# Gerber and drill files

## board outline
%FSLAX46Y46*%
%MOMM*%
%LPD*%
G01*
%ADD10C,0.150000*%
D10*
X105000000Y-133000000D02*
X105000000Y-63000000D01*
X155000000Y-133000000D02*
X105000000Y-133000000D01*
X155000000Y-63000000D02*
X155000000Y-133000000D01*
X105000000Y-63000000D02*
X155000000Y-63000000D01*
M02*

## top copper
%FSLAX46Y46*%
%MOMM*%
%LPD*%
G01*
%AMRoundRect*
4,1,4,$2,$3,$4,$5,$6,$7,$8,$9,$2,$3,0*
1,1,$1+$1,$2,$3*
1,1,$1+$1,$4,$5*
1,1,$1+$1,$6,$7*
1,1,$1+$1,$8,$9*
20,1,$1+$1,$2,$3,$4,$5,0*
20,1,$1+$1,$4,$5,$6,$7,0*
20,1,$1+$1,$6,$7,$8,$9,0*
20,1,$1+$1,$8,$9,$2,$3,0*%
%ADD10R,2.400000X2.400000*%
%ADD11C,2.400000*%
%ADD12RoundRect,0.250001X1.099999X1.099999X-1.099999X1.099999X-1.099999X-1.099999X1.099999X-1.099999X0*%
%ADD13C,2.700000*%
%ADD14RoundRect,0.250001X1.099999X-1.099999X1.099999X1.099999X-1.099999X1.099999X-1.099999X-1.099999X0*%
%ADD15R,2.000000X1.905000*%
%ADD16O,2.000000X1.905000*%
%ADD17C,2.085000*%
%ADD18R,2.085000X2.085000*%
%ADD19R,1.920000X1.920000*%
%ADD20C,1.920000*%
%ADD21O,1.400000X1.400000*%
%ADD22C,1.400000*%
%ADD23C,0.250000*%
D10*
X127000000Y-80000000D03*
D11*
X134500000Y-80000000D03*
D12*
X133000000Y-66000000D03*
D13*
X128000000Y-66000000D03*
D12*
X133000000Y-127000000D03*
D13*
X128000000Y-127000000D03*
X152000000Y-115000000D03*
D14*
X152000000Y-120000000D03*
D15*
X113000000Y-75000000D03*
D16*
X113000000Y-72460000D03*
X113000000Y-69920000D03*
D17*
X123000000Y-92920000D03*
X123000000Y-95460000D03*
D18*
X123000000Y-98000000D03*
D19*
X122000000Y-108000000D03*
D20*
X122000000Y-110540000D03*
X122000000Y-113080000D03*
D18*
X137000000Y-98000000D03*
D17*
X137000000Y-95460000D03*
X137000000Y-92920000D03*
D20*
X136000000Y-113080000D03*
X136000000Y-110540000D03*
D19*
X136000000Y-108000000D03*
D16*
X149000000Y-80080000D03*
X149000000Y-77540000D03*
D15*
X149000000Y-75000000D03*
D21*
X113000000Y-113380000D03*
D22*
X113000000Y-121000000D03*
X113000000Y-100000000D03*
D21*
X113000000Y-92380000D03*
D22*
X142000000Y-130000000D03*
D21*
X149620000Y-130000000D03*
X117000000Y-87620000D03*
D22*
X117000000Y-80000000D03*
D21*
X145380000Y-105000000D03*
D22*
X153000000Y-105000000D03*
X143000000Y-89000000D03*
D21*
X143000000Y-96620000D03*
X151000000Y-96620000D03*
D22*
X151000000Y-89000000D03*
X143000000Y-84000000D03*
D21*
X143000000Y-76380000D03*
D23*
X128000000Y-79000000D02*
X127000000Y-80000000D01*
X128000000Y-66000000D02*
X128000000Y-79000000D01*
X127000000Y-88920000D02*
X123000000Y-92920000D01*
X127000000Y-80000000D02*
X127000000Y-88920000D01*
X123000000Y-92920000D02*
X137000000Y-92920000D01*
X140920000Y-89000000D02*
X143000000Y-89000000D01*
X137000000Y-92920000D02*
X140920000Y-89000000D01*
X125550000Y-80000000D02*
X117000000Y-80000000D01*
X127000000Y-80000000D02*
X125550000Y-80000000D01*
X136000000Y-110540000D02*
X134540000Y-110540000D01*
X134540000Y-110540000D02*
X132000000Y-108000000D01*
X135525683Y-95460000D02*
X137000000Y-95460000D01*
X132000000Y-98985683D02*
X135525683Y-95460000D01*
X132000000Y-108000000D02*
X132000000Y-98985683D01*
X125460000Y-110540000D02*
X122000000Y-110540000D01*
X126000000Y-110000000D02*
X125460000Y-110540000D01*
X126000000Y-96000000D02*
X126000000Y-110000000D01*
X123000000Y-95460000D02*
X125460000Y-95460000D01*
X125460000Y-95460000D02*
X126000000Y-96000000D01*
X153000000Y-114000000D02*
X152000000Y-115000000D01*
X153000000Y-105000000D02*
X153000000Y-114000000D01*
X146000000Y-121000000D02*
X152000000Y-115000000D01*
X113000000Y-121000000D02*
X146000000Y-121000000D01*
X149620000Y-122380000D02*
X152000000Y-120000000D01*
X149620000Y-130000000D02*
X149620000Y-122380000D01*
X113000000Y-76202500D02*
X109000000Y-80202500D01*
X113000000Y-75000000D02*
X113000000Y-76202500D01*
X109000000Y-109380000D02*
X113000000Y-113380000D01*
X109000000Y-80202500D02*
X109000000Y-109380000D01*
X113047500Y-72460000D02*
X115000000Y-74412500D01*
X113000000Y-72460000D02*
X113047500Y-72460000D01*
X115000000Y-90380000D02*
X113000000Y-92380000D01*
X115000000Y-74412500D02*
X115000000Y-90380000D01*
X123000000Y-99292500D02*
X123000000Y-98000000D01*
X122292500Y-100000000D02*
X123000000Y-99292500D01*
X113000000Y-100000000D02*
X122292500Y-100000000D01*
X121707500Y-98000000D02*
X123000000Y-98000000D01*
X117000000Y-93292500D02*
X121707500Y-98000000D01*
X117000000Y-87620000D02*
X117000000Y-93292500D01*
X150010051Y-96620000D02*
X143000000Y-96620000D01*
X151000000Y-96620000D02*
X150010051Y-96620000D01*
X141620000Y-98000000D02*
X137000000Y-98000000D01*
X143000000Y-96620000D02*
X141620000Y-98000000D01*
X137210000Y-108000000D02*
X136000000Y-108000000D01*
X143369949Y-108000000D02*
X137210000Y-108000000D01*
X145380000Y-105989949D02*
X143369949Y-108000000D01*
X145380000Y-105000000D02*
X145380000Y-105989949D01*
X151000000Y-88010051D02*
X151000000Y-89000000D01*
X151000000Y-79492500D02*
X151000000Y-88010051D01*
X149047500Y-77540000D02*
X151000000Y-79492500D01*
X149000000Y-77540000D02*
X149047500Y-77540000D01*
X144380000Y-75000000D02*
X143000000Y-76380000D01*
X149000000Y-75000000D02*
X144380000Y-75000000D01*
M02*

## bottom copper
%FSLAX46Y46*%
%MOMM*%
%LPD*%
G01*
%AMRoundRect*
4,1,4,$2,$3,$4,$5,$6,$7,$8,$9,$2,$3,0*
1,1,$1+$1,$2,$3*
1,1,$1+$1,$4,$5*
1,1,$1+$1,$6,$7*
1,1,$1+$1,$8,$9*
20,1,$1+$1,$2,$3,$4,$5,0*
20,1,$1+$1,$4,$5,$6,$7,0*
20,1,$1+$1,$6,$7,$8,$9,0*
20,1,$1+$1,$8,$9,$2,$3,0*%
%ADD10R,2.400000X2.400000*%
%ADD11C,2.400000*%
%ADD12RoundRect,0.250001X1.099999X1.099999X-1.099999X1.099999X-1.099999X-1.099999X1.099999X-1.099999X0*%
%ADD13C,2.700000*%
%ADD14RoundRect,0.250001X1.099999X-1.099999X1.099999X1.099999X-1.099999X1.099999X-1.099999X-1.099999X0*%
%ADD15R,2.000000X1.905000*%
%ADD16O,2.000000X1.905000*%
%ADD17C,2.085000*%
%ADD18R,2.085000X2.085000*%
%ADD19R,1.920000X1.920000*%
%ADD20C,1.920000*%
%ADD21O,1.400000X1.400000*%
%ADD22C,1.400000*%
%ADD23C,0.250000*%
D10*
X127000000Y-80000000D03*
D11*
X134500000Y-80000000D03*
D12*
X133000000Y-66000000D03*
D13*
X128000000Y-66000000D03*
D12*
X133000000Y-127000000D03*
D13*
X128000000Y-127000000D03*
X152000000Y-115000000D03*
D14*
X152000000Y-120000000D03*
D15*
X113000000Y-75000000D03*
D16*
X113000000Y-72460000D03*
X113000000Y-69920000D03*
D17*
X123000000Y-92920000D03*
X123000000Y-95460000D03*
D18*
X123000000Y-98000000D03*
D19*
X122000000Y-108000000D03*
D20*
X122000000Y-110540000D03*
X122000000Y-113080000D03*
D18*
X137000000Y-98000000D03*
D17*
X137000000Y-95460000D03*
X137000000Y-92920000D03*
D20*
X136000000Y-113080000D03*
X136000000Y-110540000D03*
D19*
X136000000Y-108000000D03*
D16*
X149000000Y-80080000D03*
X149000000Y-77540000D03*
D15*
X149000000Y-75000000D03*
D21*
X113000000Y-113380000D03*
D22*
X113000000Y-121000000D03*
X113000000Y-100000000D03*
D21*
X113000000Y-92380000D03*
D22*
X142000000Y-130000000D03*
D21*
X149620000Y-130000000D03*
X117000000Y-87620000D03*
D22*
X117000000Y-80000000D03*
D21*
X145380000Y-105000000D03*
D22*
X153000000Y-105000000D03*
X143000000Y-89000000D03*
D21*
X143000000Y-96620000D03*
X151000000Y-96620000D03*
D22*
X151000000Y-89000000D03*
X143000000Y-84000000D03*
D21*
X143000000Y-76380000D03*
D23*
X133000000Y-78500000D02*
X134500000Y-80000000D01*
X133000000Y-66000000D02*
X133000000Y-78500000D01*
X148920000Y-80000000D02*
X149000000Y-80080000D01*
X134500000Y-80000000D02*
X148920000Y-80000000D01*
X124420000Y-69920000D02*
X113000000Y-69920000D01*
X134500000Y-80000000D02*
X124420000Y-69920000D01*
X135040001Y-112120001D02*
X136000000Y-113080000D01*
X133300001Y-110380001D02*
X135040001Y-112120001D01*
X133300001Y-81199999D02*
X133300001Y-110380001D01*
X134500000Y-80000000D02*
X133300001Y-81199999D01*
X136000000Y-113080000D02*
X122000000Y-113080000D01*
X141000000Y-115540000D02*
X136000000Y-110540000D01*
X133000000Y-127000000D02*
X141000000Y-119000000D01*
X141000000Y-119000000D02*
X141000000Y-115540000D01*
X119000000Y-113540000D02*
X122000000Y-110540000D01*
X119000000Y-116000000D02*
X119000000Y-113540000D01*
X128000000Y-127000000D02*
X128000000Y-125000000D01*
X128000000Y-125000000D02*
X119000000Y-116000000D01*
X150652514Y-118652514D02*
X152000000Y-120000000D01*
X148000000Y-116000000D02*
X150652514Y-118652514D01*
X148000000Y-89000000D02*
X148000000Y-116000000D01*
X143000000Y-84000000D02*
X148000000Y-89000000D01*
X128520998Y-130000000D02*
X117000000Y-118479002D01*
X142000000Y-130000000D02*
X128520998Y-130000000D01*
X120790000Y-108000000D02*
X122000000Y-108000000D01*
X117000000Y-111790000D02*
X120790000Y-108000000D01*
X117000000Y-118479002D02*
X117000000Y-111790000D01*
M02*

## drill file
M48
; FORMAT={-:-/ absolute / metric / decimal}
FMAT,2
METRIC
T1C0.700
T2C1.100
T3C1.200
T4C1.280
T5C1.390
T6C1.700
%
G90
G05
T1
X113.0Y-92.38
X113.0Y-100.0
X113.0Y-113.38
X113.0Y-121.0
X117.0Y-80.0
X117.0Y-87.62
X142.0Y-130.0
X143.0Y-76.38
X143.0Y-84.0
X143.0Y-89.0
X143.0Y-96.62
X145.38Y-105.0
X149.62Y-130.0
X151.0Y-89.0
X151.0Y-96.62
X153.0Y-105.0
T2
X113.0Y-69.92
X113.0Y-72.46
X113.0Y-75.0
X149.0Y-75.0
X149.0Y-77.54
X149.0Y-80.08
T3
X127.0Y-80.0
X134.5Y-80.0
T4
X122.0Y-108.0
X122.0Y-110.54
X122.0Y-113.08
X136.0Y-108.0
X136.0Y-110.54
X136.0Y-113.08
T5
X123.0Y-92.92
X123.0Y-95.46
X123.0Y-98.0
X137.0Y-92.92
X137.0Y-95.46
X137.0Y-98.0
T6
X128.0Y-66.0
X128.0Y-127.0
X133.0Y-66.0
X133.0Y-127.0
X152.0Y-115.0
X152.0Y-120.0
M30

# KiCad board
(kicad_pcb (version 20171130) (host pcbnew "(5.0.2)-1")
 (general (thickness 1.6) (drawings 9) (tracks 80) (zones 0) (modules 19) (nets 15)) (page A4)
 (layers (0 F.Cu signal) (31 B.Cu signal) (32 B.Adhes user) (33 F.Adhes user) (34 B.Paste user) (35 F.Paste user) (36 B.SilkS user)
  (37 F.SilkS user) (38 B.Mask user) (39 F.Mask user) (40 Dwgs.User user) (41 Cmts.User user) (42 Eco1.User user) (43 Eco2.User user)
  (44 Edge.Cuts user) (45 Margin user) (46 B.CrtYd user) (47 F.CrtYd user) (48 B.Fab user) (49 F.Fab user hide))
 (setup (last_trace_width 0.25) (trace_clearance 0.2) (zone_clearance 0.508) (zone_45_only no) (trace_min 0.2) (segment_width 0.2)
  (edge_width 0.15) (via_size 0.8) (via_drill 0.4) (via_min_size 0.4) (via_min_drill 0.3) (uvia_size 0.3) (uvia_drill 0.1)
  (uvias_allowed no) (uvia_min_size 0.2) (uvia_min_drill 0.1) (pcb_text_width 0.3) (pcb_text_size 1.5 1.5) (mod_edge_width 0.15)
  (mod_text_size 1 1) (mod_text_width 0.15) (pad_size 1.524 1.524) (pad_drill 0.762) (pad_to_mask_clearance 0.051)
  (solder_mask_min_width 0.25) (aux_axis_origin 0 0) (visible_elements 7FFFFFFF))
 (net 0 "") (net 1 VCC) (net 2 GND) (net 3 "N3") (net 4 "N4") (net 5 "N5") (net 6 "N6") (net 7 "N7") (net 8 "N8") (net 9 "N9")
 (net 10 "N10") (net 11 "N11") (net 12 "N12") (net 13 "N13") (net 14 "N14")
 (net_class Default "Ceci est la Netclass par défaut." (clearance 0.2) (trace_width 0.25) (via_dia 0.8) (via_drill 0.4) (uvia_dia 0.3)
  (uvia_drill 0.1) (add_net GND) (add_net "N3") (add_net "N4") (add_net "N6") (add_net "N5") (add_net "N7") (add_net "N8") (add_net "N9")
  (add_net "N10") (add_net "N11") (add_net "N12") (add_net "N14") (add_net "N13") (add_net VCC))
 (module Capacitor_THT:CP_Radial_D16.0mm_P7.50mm (layer F.Cu) (at 127 80)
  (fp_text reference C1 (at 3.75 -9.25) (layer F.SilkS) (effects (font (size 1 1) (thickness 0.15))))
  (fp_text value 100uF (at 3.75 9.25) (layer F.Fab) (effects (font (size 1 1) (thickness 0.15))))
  (pad 1 thru_hole rect (at 0 0) (size 2.4 2.4) (drill 1.2) (layers *.Cu *.Mask) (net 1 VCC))
  (pad 2 thru_hole circle (at 7.5 0) (size 2.4 2.4) (drill 1.2) (layers *.Cu *.Mask) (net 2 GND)))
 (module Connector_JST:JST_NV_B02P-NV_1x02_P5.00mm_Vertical (layer F.Cu) (at 133 66 180)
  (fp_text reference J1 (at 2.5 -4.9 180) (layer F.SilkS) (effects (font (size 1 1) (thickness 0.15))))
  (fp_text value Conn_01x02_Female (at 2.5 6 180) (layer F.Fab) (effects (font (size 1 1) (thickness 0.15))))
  (pad 1 thru_hole roundrect (at 0 0 180) (size 2.7 2.7) (drill 1.7) (layers *.Cu *.Mask) (roundrect_rratio 0.09259299999999999) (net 2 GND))
  (pad 2 thru_hole circle (at 5 0 180) (size 2.7 2.7) (drill 1.7) (layers *.Cu *.Mask) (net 1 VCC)))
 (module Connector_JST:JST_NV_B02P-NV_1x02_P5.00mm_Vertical (layer F.Cu) (at 133 127 180)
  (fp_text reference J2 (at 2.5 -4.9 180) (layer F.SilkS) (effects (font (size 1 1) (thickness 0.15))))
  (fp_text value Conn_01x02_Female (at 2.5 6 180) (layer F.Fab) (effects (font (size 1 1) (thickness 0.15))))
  (pad 1 thru_hole roundrect (at 0 0 180) (size 2.7 2.7) (drill 1.7) (layers *.Cu *.Mask) (roundrect_rratio 0.09259299999999999)
   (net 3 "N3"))
  (pad 2 thru_hole circle (at 5 0 180) (size 2.7 2.7) (drill 1.7) (layers *.Cu *.Mask) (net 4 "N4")))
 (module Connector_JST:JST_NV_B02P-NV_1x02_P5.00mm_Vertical (layer F.Cu) (at 152 120 90)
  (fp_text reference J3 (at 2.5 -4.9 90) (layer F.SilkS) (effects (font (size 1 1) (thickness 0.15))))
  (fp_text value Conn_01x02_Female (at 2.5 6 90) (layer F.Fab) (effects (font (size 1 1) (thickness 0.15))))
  (pad 2 thru_hole circle (at 5 0 90) (size 2.7 2.7) (drill 1.7) (layers *.Cu *.Mask) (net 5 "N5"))
  (pad 1 thru_hole roundrect (at 0 0 90) (size 2.7 2.7) (drill 1.7) (layers *.Cu *.Mask) (roundrect_rratio 0.09259299999999999) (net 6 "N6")))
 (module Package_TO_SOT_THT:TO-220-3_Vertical (layer F.Cu) (at 113 75 90)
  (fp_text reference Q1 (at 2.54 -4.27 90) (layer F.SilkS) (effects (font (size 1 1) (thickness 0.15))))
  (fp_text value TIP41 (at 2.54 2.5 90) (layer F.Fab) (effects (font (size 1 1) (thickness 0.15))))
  (pad 1 thru_hole rect (at 0 0 90) (size 1.905 2) (drill 1.1) (layers *.Cu *.Mask) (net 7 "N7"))
  (pad 2 thru_hole oval (at 2.54 0 90) (size 1.905 2) (drill 1.1) (layers *.Cu *.Mask) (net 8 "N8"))
  (pad 3 thru_hole oval (at 5.08 0 90) (size 1.905 2) (drill 1.1) (layers *.Cu *.Mask) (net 2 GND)))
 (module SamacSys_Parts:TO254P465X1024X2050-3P (layer F.Cu) (at 123 98 90)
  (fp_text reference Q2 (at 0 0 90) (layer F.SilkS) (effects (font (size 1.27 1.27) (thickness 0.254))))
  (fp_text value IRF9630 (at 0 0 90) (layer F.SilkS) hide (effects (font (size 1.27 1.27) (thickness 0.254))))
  (pad 3 thru_hole circle (at 5.08 0 90) (size 2.085 2.085) (drill 1.39) (layers *.Cu *.Mask) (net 1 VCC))
  (pad 2 thru_hole circle (at 2.54 0 90) (size 2.085 2.085) (drill 1.39) (layers *.Cu *.Mask) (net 4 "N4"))
  (pad 1 thru_hole rect (at 0 0 90) (size 2.085 2.085) (drill 1.39) (layers *.Cu *.Mask) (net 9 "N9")))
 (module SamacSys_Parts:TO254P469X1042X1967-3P (layer F.Cu) (at 122 108 270)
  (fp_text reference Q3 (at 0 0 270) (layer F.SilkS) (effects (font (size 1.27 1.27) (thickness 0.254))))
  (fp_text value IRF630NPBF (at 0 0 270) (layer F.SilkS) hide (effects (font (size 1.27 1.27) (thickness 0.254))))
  (pad 1 thru_hole rect (at 0 0 270) (size 1.92 1.92) (drill 1.28) (layers *.Cu *.Mask) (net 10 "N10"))
  (pad 2 thru_hole circle (at 2.54 0 270) (size 1.92 1.92) (drill 1.28) (layers *.Cu *.Mask) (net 4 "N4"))
  (pad 3 thru_hole circle (at 5.08 0 270) (size 1.92 1.92) (drill 1.28) (layers *.Cu *.Mask) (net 2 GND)))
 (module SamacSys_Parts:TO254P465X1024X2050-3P (layer F.Cu) (at 137 98 90)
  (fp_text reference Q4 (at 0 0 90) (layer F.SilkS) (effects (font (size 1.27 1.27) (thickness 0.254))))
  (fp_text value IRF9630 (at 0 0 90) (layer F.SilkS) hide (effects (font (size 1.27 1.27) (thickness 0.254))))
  (pad 1 thru_hole rect (at 0 0 90) (size 2.085 2.085) (drill 1.39) (layers *.Cu *.Mask) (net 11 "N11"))
  (pad 2 thru_hole circle (at 2.54 0 90) (size 2.085 2.085) (drill 1.39) (layers *.Cu *.Mask) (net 3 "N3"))
  (pad 3 thru_hole circle (at 5.08 0 90) (size 2.085 2.085) (drill 1.39) (layers *.Cu *.Mask) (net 1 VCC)))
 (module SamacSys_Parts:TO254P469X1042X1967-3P (layer F.Cu) (at 136 108 270)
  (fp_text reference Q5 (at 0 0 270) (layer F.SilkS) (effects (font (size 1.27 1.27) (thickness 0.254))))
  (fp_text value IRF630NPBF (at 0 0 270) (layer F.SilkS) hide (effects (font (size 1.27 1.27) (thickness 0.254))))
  (pad 3 thru_hole circle (at 5.08 0 270) (size 1.92 1.92) (drill 1.28) (layers *.Cu *.Mask) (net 2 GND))
  (pad 2 thru_hole circle (at 2.54 0 270) (size 1.92 1.92) (drill 1.28) (layers *.Cu *.Mask) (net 3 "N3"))
  (pad 1 thru_hole rect (at 0 0 270) (size 1.92 1.92) (drill 1.28) (layers *.Cu *.Mask) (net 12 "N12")))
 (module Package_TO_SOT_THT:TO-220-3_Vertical (layer F.Cu) (at 149 75 270)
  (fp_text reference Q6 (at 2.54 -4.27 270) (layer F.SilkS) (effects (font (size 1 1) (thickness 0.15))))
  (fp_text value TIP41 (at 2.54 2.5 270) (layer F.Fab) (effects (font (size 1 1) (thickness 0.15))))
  (pad 3 thru_hole oval (at 5.08 0 270) (size 1.905 2) (drill 1.1) (layers *.Cu *.Mask) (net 2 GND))
  (pad 2 thru_hole oval (at 2.54 0 270) (size 1.905 2) (drill 1.1) (layers *.Cu *.Mask) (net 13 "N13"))
  (pad 1 thru_hole rect (at 0 0 270) (size 1.905 2) (drill 1.1) (layers *.Cu *.Mask) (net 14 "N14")))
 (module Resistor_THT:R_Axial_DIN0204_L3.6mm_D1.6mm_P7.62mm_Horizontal (layer F.Cu) (at 113 121 90)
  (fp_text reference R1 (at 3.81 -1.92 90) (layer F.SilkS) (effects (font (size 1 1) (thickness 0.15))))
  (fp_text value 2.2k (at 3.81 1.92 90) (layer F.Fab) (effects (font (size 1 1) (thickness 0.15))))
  (pad 2 thru_hole oval (at 7.62 0 90) (size 1.4 1.4) (drill 0.7) (layers *.Cu *.Mask) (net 7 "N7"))
  (pad 1 thru_hole circle (at 0 0 90) (size 1.4 1.4) (drill 0.7) (layers *.Cu *.Mask) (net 5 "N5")))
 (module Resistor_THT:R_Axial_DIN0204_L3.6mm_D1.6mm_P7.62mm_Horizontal (layer F.Cu) (at 113 100 90)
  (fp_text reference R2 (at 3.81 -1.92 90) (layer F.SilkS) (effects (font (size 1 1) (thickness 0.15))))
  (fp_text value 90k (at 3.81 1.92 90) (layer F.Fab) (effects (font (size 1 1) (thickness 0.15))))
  (pad 1 thru_hole circle (at 0 0 90) (size 1.4 1.4) (drill 0.7) (layers *.Cu *.Mask) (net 9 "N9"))
  (pad 2 thru_hole oval (at 7.62 0 90) (size 1.4 1.4) (drill 0.7) (layers *.Cu *.Mask) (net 8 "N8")))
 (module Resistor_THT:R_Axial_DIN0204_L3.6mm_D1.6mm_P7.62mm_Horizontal (layer F.Cu) (at 142 130)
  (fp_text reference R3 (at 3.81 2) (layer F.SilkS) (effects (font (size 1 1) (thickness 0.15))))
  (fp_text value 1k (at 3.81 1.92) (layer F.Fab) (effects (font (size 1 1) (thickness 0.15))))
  (pad 1 thru_hole circle (at 0 0) (size 1.4 1.4) (drill 0.7) (layers *.Cu *.Mask) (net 10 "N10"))
  (pad 2 thru_hole oval (at 7.62 0) (size 1.4 1.4) (drill 0.7) (layers *.Cu *.Mask) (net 6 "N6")))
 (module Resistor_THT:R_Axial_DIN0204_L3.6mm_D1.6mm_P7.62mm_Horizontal (layer F.Cu) (at 117 80 270)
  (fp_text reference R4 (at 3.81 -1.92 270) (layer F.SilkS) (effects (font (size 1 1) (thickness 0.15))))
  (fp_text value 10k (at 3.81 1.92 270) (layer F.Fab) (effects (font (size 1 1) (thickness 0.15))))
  (pad 2 thru_hole oval (at 7.62 0 270) (size 1.4 1.4) (drill 0.7) (layers *.Cu *.Mask) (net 9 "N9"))
  (pad 1 thru_hole circle (at 0 0 270) (size 1.4 1.4) (drill 0.7) (layers *.Cu *.Mask) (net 1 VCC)))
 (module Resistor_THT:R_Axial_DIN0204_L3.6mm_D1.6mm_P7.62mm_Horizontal (layer F.Cu) (at 153 105 180)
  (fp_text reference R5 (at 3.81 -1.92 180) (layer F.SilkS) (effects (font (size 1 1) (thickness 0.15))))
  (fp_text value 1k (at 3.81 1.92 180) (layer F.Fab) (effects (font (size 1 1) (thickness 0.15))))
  (pad 2 thru_hole oval (at 7.62 0 180) (size 1.4 1.4) (drill 0.7) (layers *.Cu *.Mask) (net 12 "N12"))
  (pad 1 thru_hole circle (at 0 0 180) (size 1.4 1.4) (drill 0.7) (layers *.Cu *.Mask) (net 5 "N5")))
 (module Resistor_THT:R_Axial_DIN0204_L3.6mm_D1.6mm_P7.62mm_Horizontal (layer F.Cu) (at 143 89 270)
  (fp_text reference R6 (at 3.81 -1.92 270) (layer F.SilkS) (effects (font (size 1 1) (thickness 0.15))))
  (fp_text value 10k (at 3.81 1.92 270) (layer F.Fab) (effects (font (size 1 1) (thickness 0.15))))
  (pad 1 thru_hole circle (at 0 0 270) (size 1.4 1.4) (drill 0.7) (layers *.Cu *.Mask) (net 1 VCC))
  (pad 2 thru_hole oval (at 7.62 0 270) (size 1.4 1.4) (drill 0.7) (layers *.Cu *.Mask) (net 11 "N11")))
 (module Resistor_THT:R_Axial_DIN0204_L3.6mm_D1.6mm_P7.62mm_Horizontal (layer F.Cu) (at 151 89 270)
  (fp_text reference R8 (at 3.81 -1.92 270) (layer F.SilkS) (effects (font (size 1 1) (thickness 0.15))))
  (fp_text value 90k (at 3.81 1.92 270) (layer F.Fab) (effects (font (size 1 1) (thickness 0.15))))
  (pad 2 thru_hole oval (at 7.62 0 270) (size 1.4 1.4) (drill 0.7) (layers *.Cu *.Mask) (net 11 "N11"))
  (pad 1 thru_hole circle (at 0 0 270) (size 1.4 1.4) (drill 0.7) (layers *.Cu *.Mask) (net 13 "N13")))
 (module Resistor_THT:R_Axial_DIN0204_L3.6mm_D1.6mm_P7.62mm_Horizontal (layer F.Cu) (at 143 84 90)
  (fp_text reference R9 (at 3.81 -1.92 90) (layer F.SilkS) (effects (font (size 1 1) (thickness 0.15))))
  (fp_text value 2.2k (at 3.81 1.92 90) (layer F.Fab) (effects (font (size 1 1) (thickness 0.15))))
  (pad 1 thru_hole circle (at 0 0 90) (size 1.4 1.4) (drill 0.7) (layers *.Cu *.Mask) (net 6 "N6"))
  (pad 2 thru_hole oval (at 7.62 0 90) (size 1.4 1.4) (drill 0.7) (layers *.Cu *.Mask) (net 14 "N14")))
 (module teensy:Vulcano (layer F.Cu) (at 125 127)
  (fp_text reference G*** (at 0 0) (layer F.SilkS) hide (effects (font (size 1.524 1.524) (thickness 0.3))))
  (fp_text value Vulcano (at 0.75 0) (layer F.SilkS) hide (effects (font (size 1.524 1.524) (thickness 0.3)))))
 (gr_line (start 105 133) (end 105 63) (layer Edge.Cuts) (width 0.15))
 (gr_line (start 155 133) (end 105 133) (layer Edge.Cuts) (width 0.15))
 (gr_line (start 155 63) (end 155 133) (layer Edge.Cuts) (width 0.15))
 (gr_line (start 105 63) (end 155 63) (layer Edge.Cuts) (width 0.15))
 (segment (start 128 79) (end 127 80) (width 0.25) (layer F.Cu) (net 1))
 (segment (start 128 66) (end 128 79) (width 0.25) (layer F.Cu) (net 1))
 (segment (start 127 88.92) (end 123 92.92) (width 0.25) (layer F.Cu) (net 1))
 (segment (start 127 80) (end 127 88.92) (width 0.25) (layer F.Cu) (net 1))
 (segment (start 123 92.92) (end 137 92.92) (width 0.25) (layer F.Cu) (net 1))
 (segment (start 140.92 89) (end 143 89) (width 0.25) (layer F.Cu) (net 1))
 (segment (start 137 92.92) (end 140.92 89) (width 0.25) (layer F.Cu) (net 1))
 (segment (start 125.55 80) (end 117 80) (width 0.25) (layer F.Cu) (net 1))
 (segment (start 127 80) (end 125.55 80) (width 0.25) (layer F.Cu) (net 1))
 (segment (start 133 78.5) (end 134.5 80) (width 0.25) (layer B.Cu) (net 2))
 (segment (start 133 66) (end 133 78.5) (width 0.25) (layer B.Cu) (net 2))
 (segment (start 148.92 80) (end 149 80.08) (width 0.25) (layer B.Cu) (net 2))
 (segment (start 134.5 80) (end 148.92 80) (width 0.25) (layer B.Cu) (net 2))
 (segment (start 124.42 69.92) (end 113 69.92) (width 0.25) (layer B.Cu) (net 2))
 (segment (start 134.5 80) (end 124.42 69.92) (width 0.25) (layer B.Cu) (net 2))
 (segment (start 135.040001 112.120001) (end 136 113.08) (width 0.25) (layer B.Cu) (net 2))
 (segment (start 133.300001 110.380001) (end 135.040001 112.120001) (width 0.25) (layer B.Cu) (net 2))
 (segment (start 133.300001 81.199999) (end 133.300001 110.380001) (width 0.25) (layer B.Cu) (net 2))
 (segment (start 134.5 80) (end 133.300001 81.199999) (width 0.25) (layer B.Cu) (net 2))
 (segment (start 136 113.08) (end 122 113.08) (width 0.25) (layer B.Cu) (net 2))
 (segment (start 136 110.54) (end 134.54 110.54) (width 0.25) (layer F.Cu) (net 3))
 (segment (start 134.54 110.54) (end 132 108) (width 0.25) (layer F.Cu) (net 3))
 (segment (start 135.525683 95.46) (end 137 95.46) (width 0.25) (layer F.Cu) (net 3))
 (segment (start 132 98.985683) (end 135.525683 95.46) (width 0.25) (layer F.Cu) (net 3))
 (segment (start 132 108) (end 132 98.985683) (width 0.25) (layer F.Cu) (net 3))
 (segment (start 141 115.54) (end 136 110.54) (width 0.25) (layer B.Cu) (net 3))
 (segment (start 133 127) (end 141 119) (width 0.25) (layer B.Cu) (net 3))
 (segment (start 141 119) (end 141 115.54) (width 0.25) (layer B.Cu) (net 3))
 (segment (start 125.46 110.54) (end 122 110.54) (width 0.25) (layer F.Cu) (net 4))
 (segment (start 126 110) (end 125.46 110.54) (width 0.25) (layer F.Cu) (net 4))
 (segment (start 126 96) (end 126 110) (width 0.25) (layer F.Cu) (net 4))
 (segment (start 123 95.46) (end 125.46 95.46) (width 0.25) (layer F.Cu) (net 4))
 (segment (start 125.46 95.46) (end 126 96) (width 0.25) (layer F.Cu) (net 4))
 (segment (start 119 113.54) (end 122 110.54) (width 0.25) (layer B.Cu) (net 4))
 (segment (start 119 116) (end 119 113.54) (width 0.25) (layer B.Cu) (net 4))
 (segment (start 128 127) (end 128 125) (width 0.25) (layer B.Cu) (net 4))
 (segment (start 128 125) (end 119 116) (width 0.25) (layer B.Cu) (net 4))
 (segment (start 153 114) (end 152 115) (width 0.25) (layer F.Cu) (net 5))
 (segment (start 153 105) (end 153 114) (width 0.25) (layer F.Cu) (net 5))
 (segment (start 146 121) (end 152 115) (width 0.25) (layer F.Cu) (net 5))
 (segment (start 113 121) (end 146 121) (width 0.25) (layer F.Cu) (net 5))
 (segment (start 149.62 122.38) (end 152 120) (width 0.25) (layer F.Cu) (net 6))
 (segment (start 149.62 130) (end 149.62 122.38) (width 0.25) (layer F.Cu) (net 6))
 (segment (start 150.652514 118.652514) (end 152 120) (width 0.25) (layer B.Cu) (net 6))
 (segment (start 148 116) (end 150.652514 118.652514) (width 0.25) (layer B.Cu) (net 6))
 (segment (start 148 89) (end 148 116) (width 0.25) (layer B.Cu) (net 6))
 (segment (start 143 84) (end 148 89) (width 0.25) (layer B.Cu) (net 6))
 (segment (start 113 76.2025) (end 109 80.2025) (width 0.25) (layer F.Cu) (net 7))
 (segment (start 113 75) (end 113 76.2025) (width 0.25) (layer F.Cu) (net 7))
 (segment (start 109 109.38) (end 113 113.38) (width 0.25) (layer F.Cu) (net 7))
 (segment (start 109 80.2025) (end 109 109.38) (width 0.25) (layer F.Cu) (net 7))
 (segment (start 113.0475 72.46) (end 115 74.4125) (width 0.25) (layer F.Cu) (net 8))
 (segment (start 113 72.46) (end 113.0475 72.46) (width 0.25) (layer F.Cu) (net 8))
 (segment (start 115 90.38) (end 113 92.38) (width 0.25) (layer F.Cu) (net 8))
 (segment (start 115 74.4125) (end 115 90.38) (width 0.25) (layer F.Cu) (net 8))
 (segment (start 123 99.2925) (end 123 98) (width 0.25) (layer F.Cu) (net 9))
 (segment (start 122.2925 100) (end 123 99.2925) (width 0.25) (layer F.Cu) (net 9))
 (segment (start 113 100) (end 122.2925 100) (width 0.25) (layer F.Cu) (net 9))
 (segment (start 121.7075 98) (end 123 98) (width 0.25) (layer F.Cu) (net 9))
 (segment (start 117 93.2925) (end 121.7075 98) (width 0.25) (layer F.Cu) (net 9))
 (segment (start 117 87.62) (end 117 93.2925) (width 0.25) (layer F.Cu) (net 9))
 (segment (start 128.520998 130) (end 117 118.479002) (width 0.25) (layer B.Cu) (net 10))
 (segment (start 142 130) (end 128.520998 130) (width 0.25) (layer B.Cu) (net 10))
 (segment (start 120.79 108) (end 122 108) (width 0.25) (layer B.Cu) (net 10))
 (segment (start 117 111.79) (end 120.79 108) (width 0.25) (layer B.Cu) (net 10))
 (segment (start 117 118.479002) (end 117 111.79) (width 0.25) (layer B.Cu) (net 10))
 (segment (start 150.010051 96.62) (end 143 96.62) (width 0.25) (layer F.Cu) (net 11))
 (segment (start 151 96.62) (end 150.010051 96.62) (width 0.25) (layer F.Cu) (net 11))
 (segment (start 141.62 98) (end 137 98) (width 0.25) (layer F.Cu) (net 11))
 (segment (start 143 96.62) (end 141.62 98) (width 0.25) (layer F.Cu) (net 11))
 (segment (start 137.21 108) (end 136 108) (width 0.25) (layer F.Cu) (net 12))
 (segment (start 143.369949 108) (end 137.21 108) (width 0.25) (layer F.Cu) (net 12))
 (segment (start 145.38 105.989949) (end 143.369949 108) (width 0.25) (layer F.Cu) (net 12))
 (segment (start 145.38 105) (end 145.38 105.989949) (width 0.25) (layer F.Cu) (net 12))
 (segment (start 151 88.010051) (end 151 89) (width 0.25) (layer F.Cu) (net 13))
 (segment (start 151 79.4925) (end 151 88.010051) (width 0.25) (layer F.Cu) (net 13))
 (segment (start 149.0475 77.54) (end 151 79.4925) (width 0.25) (layer F.Cu) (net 13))
 (segment (start 149 77.54) (end 149.0475 77.54) (width 0.25) (layer F.Cu) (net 13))
 (segment (start 144.38 75) (end 143 76.38) (width 0.25) (layer F.Cu) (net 14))
 (segment (start 149 75) (end 144.38 75) (width 0.25) (layer F.Cu) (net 14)))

